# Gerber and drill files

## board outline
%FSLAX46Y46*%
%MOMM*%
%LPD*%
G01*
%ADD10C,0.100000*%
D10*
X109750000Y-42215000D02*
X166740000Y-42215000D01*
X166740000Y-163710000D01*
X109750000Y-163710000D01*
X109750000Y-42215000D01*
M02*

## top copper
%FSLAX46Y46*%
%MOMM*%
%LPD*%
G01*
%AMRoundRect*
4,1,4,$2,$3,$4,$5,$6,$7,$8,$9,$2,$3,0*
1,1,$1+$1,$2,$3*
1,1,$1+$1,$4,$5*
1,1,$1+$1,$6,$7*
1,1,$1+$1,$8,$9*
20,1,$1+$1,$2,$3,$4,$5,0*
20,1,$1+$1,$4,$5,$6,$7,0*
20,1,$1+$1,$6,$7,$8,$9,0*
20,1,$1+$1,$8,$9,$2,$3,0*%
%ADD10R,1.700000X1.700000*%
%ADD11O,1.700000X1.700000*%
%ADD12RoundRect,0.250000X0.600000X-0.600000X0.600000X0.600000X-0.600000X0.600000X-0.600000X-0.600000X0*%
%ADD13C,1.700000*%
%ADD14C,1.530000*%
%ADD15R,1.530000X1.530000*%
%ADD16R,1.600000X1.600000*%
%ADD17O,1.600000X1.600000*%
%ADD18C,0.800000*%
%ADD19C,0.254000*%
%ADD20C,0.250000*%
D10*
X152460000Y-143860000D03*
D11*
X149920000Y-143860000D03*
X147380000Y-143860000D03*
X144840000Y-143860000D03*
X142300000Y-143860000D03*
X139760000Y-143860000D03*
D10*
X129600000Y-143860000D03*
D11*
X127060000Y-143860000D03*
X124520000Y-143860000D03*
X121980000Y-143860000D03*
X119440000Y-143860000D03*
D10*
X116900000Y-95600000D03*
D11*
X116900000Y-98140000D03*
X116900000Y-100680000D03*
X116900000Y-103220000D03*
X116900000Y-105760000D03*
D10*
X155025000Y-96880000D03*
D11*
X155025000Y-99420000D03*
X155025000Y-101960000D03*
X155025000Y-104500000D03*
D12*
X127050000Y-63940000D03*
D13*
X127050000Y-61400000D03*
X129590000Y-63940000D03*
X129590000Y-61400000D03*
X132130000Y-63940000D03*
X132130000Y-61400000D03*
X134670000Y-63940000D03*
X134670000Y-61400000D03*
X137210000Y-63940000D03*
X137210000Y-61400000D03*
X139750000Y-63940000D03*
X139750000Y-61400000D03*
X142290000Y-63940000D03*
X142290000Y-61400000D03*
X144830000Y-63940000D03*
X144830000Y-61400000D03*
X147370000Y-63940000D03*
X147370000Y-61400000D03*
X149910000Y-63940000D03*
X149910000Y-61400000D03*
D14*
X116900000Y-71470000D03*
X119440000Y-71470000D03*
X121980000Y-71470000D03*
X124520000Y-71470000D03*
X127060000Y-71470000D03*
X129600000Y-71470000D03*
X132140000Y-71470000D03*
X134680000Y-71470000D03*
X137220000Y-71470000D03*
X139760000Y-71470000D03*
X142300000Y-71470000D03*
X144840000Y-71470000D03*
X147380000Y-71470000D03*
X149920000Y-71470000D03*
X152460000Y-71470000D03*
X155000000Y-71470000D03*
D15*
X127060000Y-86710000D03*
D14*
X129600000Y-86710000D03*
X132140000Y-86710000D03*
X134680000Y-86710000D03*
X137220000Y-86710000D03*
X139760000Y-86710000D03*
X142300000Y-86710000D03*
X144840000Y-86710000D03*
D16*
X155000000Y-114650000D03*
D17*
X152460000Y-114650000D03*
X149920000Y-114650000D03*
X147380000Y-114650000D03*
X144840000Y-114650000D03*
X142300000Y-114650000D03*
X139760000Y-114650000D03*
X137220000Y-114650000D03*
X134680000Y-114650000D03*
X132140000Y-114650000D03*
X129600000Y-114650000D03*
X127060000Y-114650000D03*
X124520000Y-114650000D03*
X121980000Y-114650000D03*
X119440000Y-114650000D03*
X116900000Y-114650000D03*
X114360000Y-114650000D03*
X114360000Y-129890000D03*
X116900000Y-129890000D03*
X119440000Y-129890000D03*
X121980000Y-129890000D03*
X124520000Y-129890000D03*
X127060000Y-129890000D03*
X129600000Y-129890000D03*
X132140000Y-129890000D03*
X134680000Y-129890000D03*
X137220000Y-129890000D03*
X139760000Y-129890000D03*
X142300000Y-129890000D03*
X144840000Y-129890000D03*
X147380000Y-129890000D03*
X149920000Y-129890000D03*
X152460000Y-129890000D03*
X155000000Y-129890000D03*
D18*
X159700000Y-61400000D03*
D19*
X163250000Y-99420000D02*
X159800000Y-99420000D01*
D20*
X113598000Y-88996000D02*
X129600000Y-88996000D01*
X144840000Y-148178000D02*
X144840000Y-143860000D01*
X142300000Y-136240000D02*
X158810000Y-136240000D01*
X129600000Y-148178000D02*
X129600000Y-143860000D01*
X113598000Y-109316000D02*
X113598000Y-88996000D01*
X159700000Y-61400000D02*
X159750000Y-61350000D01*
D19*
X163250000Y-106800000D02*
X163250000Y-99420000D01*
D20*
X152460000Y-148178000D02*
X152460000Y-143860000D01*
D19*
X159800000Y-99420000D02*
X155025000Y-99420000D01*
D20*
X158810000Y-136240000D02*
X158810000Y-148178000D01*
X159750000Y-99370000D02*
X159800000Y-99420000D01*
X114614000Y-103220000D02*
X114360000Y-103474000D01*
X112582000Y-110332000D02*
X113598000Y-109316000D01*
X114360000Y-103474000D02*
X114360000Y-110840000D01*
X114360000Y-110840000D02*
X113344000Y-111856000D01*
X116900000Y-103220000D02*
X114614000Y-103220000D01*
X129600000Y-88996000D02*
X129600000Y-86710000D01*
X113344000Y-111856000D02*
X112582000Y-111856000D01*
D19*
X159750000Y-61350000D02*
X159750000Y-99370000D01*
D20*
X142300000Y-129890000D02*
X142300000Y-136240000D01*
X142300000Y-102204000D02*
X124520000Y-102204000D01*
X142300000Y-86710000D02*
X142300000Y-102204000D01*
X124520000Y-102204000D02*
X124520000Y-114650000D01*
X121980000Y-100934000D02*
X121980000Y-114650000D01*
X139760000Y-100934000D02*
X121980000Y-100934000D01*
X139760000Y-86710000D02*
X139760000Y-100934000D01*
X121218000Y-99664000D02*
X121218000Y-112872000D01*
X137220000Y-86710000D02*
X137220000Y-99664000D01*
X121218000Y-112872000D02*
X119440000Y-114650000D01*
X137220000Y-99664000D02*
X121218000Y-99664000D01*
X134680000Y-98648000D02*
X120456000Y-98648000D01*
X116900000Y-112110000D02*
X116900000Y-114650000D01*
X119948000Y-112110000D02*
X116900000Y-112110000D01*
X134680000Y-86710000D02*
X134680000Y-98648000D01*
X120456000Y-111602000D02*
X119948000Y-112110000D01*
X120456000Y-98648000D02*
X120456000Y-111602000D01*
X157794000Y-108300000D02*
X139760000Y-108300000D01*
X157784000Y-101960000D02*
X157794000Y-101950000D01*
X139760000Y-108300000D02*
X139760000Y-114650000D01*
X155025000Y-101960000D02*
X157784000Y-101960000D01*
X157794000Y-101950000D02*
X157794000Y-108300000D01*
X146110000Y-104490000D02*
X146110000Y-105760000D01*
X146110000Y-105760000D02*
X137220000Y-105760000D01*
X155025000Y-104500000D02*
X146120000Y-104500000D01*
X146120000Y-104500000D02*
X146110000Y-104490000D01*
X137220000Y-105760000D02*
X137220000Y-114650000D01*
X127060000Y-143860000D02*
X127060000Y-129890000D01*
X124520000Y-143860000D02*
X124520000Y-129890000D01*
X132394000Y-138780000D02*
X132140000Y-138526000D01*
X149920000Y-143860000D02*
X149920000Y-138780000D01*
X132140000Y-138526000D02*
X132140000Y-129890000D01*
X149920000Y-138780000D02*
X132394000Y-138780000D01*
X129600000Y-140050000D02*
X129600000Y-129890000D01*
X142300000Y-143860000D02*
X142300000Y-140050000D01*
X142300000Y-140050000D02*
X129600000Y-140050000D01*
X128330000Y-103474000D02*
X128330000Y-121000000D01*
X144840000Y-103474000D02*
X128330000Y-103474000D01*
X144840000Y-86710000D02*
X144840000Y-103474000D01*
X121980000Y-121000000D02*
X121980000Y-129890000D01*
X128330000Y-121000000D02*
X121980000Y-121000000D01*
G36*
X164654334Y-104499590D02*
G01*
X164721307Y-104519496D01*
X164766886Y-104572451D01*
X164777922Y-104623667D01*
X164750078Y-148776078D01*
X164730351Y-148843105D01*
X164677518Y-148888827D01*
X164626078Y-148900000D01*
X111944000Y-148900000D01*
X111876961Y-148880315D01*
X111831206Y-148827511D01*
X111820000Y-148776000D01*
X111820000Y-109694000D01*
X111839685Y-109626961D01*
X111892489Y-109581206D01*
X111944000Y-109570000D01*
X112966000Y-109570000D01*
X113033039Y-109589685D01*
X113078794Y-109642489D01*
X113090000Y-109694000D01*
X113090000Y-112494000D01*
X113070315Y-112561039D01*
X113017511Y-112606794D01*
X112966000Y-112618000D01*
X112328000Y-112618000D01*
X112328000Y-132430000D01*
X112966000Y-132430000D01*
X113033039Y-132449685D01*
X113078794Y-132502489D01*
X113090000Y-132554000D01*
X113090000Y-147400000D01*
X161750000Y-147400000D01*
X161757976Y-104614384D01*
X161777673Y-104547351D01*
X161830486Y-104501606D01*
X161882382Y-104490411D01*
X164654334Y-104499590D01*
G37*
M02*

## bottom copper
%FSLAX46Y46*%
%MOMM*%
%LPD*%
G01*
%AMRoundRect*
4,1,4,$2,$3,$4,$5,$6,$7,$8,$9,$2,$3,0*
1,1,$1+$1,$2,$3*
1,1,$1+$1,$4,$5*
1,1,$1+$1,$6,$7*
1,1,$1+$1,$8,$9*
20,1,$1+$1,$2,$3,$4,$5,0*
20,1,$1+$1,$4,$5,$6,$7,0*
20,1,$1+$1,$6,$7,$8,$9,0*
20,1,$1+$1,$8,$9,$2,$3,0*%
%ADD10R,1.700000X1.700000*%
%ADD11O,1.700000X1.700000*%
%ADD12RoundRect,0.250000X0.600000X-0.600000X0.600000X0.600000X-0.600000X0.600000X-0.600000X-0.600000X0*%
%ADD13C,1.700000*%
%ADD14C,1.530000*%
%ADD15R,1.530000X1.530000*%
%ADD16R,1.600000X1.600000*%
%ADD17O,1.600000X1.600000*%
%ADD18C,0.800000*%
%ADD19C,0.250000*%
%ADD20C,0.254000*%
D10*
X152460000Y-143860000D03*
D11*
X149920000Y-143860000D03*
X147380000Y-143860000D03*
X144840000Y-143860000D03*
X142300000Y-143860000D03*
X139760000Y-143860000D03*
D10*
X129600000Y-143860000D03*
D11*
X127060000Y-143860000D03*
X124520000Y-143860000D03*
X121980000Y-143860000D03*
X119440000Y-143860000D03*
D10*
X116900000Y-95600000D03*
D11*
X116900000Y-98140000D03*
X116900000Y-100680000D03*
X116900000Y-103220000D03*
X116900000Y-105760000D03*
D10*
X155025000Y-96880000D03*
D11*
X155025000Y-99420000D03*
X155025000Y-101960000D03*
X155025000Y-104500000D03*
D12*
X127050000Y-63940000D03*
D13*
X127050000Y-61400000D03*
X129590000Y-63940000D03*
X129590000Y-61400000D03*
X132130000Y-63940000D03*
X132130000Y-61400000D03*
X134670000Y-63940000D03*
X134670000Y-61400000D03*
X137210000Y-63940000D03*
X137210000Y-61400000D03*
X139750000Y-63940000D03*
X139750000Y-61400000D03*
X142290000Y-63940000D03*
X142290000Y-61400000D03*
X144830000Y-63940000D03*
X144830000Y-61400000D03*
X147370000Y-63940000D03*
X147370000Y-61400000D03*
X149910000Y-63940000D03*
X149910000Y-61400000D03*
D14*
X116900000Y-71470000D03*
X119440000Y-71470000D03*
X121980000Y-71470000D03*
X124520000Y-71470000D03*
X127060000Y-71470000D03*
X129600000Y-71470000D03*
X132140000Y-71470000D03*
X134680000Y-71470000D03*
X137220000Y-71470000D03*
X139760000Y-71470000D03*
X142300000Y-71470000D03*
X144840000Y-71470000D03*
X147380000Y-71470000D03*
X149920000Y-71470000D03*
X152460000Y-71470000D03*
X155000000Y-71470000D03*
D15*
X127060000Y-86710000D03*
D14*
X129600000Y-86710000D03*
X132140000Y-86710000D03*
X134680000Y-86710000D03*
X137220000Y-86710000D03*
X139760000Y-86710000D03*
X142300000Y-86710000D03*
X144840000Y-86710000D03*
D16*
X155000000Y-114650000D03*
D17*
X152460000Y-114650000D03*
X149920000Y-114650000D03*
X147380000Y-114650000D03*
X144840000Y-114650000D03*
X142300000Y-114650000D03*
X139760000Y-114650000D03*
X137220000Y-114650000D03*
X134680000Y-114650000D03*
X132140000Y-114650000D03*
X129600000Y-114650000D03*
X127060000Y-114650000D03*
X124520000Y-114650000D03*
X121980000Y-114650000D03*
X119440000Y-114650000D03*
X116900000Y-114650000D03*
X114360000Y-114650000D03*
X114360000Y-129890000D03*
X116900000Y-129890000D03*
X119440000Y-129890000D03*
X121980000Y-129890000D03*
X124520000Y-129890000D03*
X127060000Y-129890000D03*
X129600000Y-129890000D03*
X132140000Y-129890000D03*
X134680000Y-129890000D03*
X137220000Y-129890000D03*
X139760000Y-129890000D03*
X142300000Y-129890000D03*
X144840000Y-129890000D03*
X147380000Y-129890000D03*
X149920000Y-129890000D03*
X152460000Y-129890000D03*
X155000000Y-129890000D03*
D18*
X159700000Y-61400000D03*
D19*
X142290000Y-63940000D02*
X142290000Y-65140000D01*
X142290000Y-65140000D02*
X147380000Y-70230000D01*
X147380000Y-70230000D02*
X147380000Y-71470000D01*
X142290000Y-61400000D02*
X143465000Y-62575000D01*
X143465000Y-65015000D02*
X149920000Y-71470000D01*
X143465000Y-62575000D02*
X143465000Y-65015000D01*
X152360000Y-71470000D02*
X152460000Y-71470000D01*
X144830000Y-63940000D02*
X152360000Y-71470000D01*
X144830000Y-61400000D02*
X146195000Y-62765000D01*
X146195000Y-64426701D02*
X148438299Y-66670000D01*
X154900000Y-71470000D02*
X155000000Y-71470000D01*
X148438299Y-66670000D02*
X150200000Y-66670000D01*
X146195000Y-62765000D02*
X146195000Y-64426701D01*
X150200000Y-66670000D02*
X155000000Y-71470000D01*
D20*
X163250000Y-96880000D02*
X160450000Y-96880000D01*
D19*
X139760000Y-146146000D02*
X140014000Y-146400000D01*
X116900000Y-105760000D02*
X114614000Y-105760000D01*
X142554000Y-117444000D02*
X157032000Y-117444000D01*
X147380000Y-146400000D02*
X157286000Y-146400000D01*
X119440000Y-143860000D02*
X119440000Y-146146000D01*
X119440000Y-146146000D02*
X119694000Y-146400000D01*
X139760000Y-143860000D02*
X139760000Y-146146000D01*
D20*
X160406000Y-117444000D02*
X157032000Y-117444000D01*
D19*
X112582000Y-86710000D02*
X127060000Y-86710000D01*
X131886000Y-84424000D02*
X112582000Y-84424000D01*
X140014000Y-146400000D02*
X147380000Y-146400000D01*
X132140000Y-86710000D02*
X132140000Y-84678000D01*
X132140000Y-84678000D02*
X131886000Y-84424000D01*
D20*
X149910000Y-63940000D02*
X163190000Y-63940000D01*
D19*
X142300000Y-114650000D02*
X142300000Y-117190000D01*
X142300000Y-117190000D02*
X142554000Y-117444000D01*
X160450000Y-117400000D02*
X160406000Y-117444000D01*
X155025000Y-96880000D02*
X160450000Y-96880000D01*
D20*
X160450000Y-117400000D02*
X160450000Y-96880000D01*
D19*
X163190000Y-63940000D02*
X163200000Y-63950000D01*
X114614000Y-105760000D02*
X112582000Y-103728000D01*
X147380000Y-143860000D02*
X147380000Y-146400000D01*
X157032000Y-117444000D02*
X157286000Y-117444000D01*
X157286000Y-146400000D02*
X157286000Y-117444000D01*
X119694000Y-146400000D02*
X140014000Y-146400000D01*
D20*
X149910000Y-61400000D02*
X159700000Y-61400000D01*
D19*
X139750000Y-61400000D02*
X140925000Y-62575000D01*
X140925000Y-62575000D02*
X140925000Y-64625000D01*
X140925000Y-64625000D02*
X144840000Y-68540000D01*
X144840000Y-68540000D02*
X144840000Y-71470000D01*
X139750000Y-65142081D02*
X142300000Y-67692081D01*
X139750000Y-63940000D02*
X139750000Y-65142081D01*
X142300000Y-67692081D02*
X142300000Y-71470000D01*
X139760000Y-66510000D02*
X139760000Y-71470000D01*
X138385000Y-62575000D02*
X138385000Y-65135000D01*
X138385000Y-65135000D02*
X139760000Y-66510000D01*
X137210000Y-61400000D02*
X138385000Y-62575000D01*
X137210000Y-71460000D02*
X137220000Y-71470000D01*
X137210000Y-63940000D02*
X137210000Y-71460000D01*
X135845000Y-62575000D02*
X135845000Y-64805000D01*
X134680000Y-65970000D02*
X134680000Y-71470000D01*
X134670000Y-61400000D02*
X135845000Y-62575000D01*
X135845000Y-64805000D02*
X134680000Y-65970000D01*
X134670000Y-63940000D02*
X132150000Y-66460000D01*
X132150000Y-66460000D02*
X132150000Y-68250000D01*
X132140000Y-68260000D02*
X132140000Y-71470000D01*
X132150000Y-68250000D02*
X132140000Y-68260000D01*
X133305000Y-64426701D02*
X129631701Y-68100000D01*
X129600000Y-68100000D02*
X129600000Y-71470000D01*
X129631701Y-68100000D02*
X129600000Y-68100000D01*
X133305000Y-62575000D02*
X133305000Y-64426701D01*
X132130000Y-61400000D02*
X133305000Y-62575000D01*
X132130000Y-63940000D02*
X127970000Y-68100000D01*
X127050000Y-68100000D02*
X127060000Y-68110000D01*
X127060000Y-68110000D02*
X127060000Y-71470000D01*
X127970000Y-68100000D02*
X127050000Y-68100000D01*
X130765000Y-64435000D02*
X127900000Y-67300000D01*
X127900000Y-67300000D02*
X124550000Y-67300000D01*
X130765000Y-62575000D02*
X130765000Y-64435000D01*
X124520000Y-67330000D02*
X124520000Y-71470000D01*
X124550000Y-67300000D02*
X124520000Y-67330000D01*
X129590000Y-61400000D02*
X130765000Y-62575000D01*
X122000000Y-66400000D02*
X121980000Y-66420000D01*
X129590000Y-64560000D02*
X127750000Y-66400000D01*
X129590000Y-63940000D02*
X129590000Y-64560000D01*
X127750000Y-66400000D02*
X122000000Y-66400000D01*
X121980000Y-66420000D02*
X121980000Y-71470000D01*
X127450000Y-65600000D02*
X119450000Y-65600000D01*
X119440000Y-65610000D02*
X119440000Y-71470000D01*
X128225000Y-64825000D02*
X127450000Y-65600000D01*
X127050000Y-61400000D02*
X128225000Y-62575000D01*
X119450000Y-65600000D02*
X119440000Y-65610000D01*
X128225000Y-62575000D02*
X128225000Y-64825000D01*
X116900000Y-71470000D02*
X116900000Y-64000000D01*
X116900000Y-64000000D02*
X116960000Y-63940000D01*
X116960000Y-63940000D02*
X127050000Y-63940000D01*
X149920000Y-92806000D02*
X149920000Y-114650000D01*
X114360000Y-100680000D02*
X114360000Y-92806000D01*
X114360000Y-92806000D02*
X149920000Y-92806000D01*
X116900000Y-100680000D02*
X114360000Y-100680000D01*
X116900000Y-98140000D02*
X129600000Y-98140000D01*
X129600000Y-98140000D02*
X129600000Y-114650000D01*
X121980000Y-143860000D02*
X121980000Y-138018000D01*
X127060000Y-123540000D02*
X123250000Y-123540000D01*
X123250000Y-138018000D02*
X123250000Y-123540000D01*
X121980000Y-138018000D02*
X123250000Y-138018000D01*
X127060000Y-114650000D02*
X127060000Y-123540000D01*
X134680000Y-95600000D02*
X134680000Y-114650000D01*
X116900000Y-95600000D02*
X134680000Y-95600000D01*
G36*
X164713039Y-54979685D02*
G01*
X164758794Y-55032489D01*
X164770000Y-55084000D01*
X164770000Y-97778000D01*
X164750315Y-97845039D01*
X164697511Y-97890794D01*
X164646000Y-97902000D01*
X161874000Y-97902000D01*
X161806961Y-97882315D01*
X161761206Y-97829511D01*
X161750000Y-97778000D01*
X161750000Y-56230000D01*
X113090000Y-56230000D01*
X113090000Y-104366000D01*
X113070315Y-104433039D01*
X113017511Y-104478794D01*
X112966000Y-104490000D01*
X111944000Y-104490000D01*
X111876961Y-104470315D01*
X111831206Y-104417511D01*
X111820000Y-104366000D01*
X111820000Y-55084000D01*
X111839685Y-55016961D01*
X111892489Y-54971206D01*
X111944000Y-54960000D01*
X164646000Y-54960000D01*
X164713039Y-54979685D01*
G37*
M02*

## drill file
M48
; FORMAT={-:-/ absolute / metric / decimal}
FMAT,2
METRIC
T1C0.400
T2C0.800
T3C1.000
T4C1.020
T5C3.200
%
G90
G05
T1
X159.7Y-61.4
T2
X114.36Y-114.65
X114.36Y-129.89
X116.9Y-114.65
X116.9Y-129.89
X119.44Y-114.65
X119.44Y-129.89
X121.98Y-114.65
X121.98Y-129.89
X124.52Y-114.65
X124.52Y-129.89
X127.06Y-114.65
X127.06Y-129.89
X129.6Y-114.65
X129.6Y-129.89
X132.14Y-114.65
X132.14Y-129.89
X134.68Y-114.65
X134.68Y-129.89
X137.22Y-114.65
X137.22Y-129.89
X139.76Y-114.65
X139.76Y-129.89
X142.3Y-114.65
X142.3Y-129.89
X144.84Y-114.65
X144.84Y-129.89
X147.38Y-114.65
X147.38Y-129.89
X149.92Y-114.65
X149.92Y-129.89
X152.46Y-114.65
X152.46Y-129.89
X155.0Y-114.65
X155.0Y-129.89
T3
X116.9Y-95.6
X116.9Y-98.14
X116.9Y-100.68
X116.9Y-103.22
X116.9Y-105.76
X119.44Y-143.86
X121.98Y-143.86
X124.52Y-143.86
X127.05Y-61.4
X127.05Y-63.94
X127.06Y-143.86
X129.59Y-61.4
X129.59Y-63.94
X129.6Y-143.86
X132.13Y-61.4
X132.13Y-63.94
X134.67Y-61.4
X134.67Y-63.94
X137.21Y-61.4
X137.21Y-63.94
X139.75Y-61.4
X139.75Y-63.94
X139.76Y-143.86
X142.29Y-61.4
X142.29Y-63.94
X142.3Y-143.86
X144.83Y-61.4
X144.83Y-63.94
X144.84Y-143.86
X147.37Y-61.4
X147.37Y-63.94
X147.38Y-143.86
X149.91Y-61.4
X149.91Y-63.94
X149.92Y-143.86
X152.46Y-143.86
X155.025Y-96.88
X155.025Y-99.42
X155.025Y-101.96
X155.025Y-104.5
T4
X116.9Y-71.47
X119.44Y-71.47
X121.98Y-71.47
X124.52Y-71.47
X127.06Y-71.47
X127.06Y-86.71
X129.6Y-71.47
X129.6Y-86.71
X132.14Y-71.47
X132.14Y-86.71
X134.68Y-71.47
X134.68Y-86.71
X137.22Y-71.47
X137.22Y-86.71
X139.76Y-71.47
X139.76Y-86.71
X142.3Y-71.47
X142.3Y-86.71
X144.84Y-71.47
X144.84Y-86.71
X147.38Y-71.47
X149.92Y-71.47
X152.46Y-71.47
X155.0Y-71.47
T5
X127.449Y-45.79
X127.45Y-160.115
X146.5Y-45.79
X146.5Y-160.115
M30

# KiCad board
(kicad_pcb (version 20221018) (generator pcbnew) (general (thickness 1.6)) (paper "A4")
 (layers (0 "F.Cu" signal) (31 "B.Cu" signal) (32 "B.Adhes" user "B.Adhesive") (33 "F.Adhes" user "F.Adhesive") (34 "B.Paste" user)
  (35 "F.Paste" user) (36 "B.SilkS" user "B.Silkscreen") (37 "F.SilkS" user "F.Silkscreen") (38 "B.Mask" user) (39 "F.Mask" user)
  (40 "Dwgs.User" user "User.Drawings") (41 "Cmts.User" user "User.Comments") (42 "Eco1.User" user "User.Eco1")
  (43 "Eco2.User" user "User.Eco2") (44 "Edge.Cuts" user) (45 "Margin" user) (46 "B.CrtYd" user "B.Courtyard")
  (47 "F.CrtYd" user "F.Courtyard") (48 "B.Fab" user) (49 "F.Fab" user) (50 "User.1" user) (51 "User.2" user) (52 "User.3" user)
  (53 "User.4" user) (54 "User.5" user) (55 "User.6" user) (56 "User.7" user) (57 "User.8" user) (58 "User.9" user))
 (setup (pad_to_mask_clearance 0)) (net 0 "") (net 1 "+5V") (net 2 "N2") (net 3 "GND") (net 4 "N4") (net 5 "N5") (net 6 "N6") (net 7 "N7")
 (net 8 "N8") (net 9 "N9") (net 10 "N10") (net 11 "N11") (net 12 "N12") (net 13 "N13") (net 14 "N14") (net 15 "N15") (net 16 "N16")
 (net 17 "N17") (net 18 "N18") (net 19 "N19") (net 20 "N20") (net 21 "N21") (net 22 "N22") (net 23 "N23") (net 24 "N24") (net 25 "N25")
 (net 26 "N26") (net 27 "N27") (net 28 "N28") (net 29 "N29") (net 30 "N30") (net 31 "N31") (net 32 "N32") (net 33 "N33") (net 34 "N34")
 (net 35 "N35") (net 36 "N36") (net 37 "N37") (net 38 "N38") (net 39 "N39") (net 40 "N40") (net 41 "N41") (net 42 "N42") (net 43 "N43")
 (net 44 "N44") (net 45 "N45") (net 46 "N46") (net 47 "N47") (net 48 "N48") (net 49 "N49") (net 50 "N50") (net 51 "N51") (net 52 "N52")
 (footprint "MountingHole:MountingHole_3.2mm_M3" (layer "F.Cu") (at 127.448582 45.79)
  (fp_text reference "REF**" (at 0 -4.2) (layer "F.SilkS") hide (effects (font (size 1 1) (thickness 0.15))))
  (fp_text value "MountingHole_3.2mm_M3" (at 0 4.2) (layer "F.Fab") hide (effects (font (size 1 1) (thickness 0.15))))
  (pad "" np_thru_hole circle (at 0 0) (size 3.2 3.2) (drill 3.2) (layers "*.Cu" "*.Mask")))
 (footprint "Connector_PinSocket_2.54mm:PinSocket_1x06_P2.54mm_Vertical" (layer "F.Cu") (at 152.46 143.86 -90)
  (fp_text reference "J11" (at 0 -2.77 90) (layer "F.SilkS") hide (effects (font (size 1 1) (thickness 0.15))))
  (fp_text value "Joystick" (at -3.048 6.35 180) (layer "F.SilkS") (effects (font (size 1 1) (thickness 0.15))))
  (pad "1" thru_hole rect (at 0 0 270) (size 1.7 1.7) (drill 1) (layers "*.Cu" "*.Mask") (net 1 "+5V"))
  (pad "2" thru_hole oval (at 0 2.54 270) (size 1.7 1.7) (drill 1) (layers "*.Cu" "*.Mask") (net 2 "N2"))
  (pad "3" thru_hole oval (at 0 5.08 270) (size 1.7 1.7) (drill 1) (layers "*.Cu" "*.Mask") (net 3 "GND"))
  (pad "4" thru_hole oval (at 0 7.62 270) (size 1.7 1.7) (drill 1) (layers "*.Cu" "*.Mask") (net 1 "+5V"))
  (pad "5" thru_hole oval (at 0 10.16 270) (size 1.7 1.7) (drill 1) (layers "*.Cu" "*.Mask") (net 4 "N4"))
  (pad "6" thru_hole oval (at 0 12.7 270) (size 1.7 1.7) (drill 1) (layers "*.Cu" "*.Mask") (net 3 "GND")))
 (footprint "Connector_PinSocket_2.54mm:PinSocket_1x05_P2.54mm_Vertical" (layer "F.Cu") (at 129.6 143.86 -90)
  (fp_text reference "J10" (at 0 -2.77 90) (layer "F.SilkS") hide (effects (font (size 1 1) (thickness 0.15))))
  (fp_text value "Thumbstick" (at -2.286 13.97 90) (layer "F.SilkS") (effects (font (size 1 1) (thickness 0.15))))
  (pad "1" thru_hole rect (at 0 0 270) (size 1.7 1.7) (drill 1) (layers "*.Cu" "*.Mask") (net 1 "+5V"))
  (pad "2" thru_hole oval (at 0 2.54 270) (size 1.7 1.7) (drill 1) (layers "*.Cu" "*.Mask") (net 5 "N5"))
  (pad "3" thru_hole oval (at 0 5.08 270) (size 1.7 1.7) (drill 1) (layers "*.Cu" "*.Mask") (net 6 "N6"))
  (pad "4" thru_hole oval (at 0 7.62 270) (size 1.7 1.7) (drill 1) (layers "*.Cu" "*.Mask") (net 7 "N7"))
  (pad "5" thru_hole oval (at 0 10.16 270) (size 1.7 1.7) (drill 1) (layers "*.Cu" "*.Mask") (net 3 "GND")))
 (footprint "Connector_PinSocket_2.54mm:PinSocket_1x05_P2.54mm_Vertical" (layer "F.Cu") (at 116.9 95.6)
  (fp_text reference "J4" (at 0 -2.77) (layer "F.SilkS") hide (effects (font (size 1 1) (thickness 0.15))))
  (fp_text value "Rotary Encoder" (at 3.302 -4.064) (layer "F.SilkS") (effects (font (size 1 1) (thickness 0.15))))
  (pad "1" thru_hole rect (at 0 0) (size 1.7 1.7) (drill 1) (layers "*.Cu" "*.Mask") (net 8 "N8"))
  (pad "2" thru_hole oval (at 0 2.54) (size 1.7 1.7) (drill 1) (layers "*.Cu" "*.Mask") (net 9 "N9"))
  (pad "3" thru_hole oval (at 0 5.08) (size 1.7 1.7) (drill 1) (layers "*.Cu" "*.Mask") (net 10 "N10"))
  (pad "4" thru_hole oval (at 0 7.62) (size 1.7 1.7) (drill 1) (layers "*.Cu" "*.Mask") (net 1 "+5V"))
  (pad "5" thru_hole oval (at 0 10.16) (size 1.7 1.7) (drill 1) (layers "*.Cu" "*.Mask") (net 3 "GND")))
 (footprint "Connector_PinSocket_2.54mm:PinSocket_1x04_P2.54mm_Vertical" (layer "F.Cu") (at 155.025 96.88)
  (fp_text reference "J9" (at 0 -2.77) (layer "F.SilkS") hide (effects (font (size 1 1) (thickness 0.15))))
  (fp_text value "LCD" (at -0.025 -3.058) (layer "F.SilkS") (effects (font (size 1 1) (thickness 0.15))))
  (pad "1" thru_hole rect (at 0 0) (size 1.7 1.7) (drill 1) (layers "*.Cu" "*.Mask") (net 3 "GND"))
  (pad "2" thru_hole oval (at 0 2.54) (size 1.7 1.7) (drill 1) (layers "*.Cu" "*.Mask") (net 1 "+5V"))
  (pad "3" thru_hole oval (at 0 5.08) (size 1.7 1.7) (drill 1) (layers "*.Cu" "*.Mask") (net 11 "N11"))
  (pad "4" thru_hole oval (at 0 7.62) (size 1.7 1.7) (drill 1) (layers "*.Cu" "*.Mask") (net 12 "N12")))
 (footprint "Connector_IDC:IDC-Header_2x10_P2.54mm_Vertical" (layer "F.Cu") (at 127.05 63.94 90)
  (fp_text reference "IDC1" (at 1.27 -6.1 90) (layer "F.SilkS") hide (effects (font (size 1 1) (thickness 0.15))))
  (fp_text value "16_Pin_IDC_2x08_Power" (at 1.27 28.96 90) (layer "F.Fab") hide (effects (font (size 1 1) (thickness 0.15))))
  (pad "1" thru_hole roundrect (at 0 0 90) (size 1.7 1.7) (drill 1) (layers "*.Cu" "*.Mask") (roundrect_rratio 0.1470588235) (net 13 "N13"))
  (pad "2" thru_hole circle (at 2.54 0 90) (size 1.7 1.7) (drill 1) (layers "*.Cu" "*.Mask") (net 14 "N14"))
  (pad "3" thru_hole circle (at 0 2.54 90) (size 1.7 1.7) (drill 1) (layers "*.Cu" "*.Mask") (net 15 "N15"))
  (pad "4" thru_hole circle (at 2.54 2.54 90) (size 1.7 1.7) (drill 1) (layers "*.Cu" "*.Mask") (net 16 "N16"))
  (pad "5" thru_hole circle (at 0 5.08 90) (size 1.7 1.7) (drill 1) (layers "*.Cu" "*.Mask") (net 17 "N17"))
  (pad "6" thru_hole circle (at 2.54 5.08 90) (size 1.7 1.7) (drill 1) (layers "*.Cu" "*.Mask") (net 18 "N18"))
  (pad "7" thru_hole circle (at 0 7.62 90) (size 1.7 1.7) (drill 1) (layers "*.Cu" "*.Mask") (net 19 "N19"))
  (pad "8" thru_hole circle (at 2.54 7.62 90) (size 1.7 1.7) (drill 1) (layers "*.Cu" "*.Mask") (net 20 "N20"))
  (pad "9" thru_hole circle (at 0 10.16 90) (size 1.7 1.7) (drill 1) (layers "*.Cu" "*.Mask") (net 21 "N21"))
  (pad "10" thru_hole circle (at 2.54 10.16 90) (size 1.7 1.7) (drill 1) (layers "*.Cu" "*.Mask") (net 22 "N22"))
  (pad "11" thru_hole circle (at 0 12.7 90) (size 1.7 1.7) (drill 1) (layers "*.Cu" "*.Mask") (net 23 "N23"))
  (pad "12" thru_hole circle (at 2.54 12.7 90) (size 1.7 1.7) (drill 1) (layers "*.Cu" "*.Mask") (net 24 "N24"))
  (pad "13" thru_hole circle (at 0 15.24 90) (size 1.7 1.7) (drill 1) (layers "*.Cu" "*.Mask") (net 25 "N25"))
  (pad "14" thru_hole circle (at 2.54 15.24 90) (size 1.7 1.7) (drill 1) (layers "*.Cu" "*.Mask") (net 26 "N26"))
  (pad "15" thru_hole circle (at 0 17.78 90) (size 1.7 1.7) (drill 1) (layers "*.Cu" "*.Mask") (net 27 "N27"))
  (pad "16" thru_hole circle (at 2.54 17.78 90) (size 1.7 1.7) (drill 1) (layers "*.Cu" "*.Mask") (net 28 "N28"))
  (pad "17" thru_hole circle (at 0 20.32 90) (size 1.7 1.7) (drill 1) (layers "*.Cu" "*.Mask") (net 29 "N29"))
  (pad "18" thru_hole circle (at 2.54 20.32 90) (size 1.7 1.7) (drill 1) (layers "*.Cu" "*.Mask") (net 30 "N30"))
  (pad "19" thru_hole circle (at 0 22.86 90) (size 1.7 1.7) (drill 1) (layers "*.Cu" "*.Mask") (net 3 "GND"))
  (pad "20" thru_hole circle (at 2.54 22.86 90) (size 1.7 1.7) (drill 1) (layers "*.Cu" "*.Mask") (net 1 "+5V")))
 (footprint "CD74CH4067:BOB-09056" (layer "F.Cu") (at 135.95 79.09 -90)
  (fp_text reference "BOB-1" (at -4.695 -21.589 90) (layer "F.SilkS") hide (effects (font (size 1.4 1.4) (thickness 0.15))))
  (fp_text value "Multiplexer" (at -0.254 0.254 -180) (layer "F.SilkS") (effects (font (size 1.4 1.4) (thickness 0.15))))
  (pad "JP1-1" thru_hole circle (at -7.62 19.05 270) (size 1.53 1.53) (drill 1.02) (layers "*.Cu" "*.Mask") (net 13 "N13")
   (solder_mask_margin 0.102))
  (pad "JP1-2" thru_hole circle (at -7.62 16.51 270) (size 1.53 1.53) (drill 1.02) (layers "*.Cu" "*.Mask") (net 14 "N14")
   (solder_mask_margin 0.102))
  (pad "JP1-3" thru_hole circle (at -7.62 13.97 270) (size 1.53 1.53) (drill 1.02) (layers "*.Cu" "*.Mask") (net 15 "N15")
   (solder_mask_margin 0.102))
  (pad "JP1-4" thru_hole circle (at -7.62 11.43 270) (size 1.53 1.53) (drill 1.02) (layers "*.Cu" "*.Mask") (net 16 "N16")
   (solder_mask_margin 0.102))
  (pad "JP1-5" thru_hole circle (at -7.62 8.89 270) (size 1.53 1.53) (drill 1.02) (layers "*.Cu" "*.Mask") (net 17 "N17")
   (solder_mask_margin 0.102))
  (pad "JP1-6" thru_hole circle (at -7.62 6.35 270) (size 1.53 1.53) (drill 1.02) (layers "*.Cu" "*.Mask") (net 18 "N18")
   (solder_mask_margin 0.102))
  (pad "JP1-7" thru_hole circle (at -7.62 3.81 270) (size 1.53 1.53) (drill 1.02) (layers "*.Cu" "*.Mask") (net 19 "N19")
   (solder_mask_margin 0.102))
  (pad "JP1-8" thru_hole circle (at -7.62 1.27 270) (size 1.53 1.53) (drill 1.02) (layers "*.Cu" "*.Mask") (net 20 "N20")
   (solder_mask_margin 0.102))
  (pad "JP1-9" thru_hole circle (at -7.62 -1.27 270) (size 1.53 1.53) (drill 1.02) (layers "*.Cu" "*.Mask") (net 21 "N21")
   (solder_mask_margin 0.102))
  (pad "JP1-10" thru_hole circle (at -7.62 -3.81 270) (size 1.53 1.53) (drill 1.02) (layers "*.Cu" "*.Mask") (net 22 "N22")
   (solder_mask_margin 0.102))
  (pad "JP1-11" thru_hole circle (at -7.62 -6.35 270) (size 1.53 1.53) (drill 1.02) (layers "*.Cu" "*.Mask") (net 23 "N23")
   (solder_mask_margin 0.102))
  (pad "JP1-12" thru_hole circle (at -7.62 -8.89 270) (size 1.53 1.53) (drill 1.02) (layers "*.Cu" "*.Mask") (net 24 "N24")
   (solder_mask_margin 0.102))
  (pad "JP1-13" thru_hole circle (at -7.62 -11.43 270) (size 1.53 1.53) (drill 1.02) (layers "*.Cu" "*.Mask") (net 25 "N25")
   (solder_mask_margin 0.102))
  (pad "JP1-14" thru_hole circle (at -7.62 -13.97 270) (size 1.53 1.53) (drill 1.02) (layers "*.Cu" "*.Mask") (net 26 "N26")
   (solder_mask_margin 0.102))
  (pad "JP1-15" thru_hole circle (at -7.62 -16.51 270) (size 1.53 1.53) (drill 1.02) (layers "*.Cu" "*.Mask") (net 27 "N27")
   (solder_mask_margin 0.102))
  (pad "JP1-16" thru_hole circle (at -7.62 -19.05 270) (size 1.53 1.53) (drill 1.02) (layers "*.Cu" "*.Mask") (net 28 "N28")
   (solder_mask_margin 0.102))
  (pad "JP3-1" thru_hole rect (at 7.62 8.89 270) (size 1.53 1.53) (drill 1.02) (layers "*.Cu" "*.Mask") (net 3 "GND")
   (solder_mask_margin 0.102))
  (pad "JP3-2" thru_hole circle (at 7.62 6.35 270) (size 1.53 1.53) (drill 1.02) (layers "*.Cu" "*.Mask") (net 1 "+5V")
   (solder_mask_margin 0.102))
  (pad "JP3-3" thru_hole circle (at 7.62 3.81 270) (size 1.53 1.53) (drill 1.02) (layers "*.Cu" "*.Mask") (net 3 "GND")
   (solder_mask_margin 0.102))
  (pad "JP3-4" thru_hole circle (at 7.62 1.27 270) (size 1.53 1.53) (drill 1.02) (layers "*.Cu" "*.Mask") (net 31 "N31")
   (solder_mask_margin 0.102))
  (pad "JP3-5" thru_hole circle (at 7.62 -1.27 270) (size 1.53 1.53) (drill 1.02) (layers "*.Cu" "*.Mask") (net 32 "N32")
   (solder_mask_margin 0.102))
  (pad "JP3-6" thru_hole circle (at 7.62 -3.81 270) (size 1.53 1.53) (drill 1.02) (layers "*.Cu" "*.Mask") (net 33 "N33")
   (solder_mask_margin 0.102))
  (pad "JP3-7" thru_hole circle (at 7.62 -6.35 270) (size 1.53 1.53) (drill 1.02) (layers "*.Cu" "*.Mask") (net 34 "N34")
   (solder_mask_margin 0.102))
  (pad "JP3-8" thru_hole circle (at 7.62 -8.89 270) (size 1.53 1.53) (drill 1.02) (layers "*.Cu" "*.Mask") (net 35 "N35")
   (solder_mask_margin 0.102)))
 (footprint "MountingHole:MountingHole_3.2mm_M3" (layer "F.Cu") (at 146.5 160.115)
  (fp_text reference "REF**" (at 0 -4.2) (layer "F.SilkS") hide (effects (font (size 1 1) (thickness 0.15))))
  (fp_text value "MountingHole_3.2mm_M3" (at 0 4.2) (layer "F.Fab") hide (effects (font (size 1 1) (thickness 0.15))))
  (pad "" np_thru_hole circle (at 0 0) (size 3.2 3.2) (drill 3.2) (layers "*.Cu" "*.Mask")))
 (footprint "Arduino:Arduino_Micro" (layer "F.Cu") (at 155 114.65 -90)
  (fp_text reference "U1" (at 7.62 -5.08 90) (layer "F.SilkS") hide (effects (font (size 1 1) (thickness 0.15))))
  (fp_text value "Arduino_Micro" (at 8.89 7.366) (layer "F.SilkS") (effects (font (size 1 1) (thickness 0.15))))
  (pad "1" thru_hole rect (at 0 0 270) (size 1.6 1.6) (drill 0.8) (layers "*.Cu" "*.Mask") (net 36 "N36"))
  (pad "2" thru_hole oval (at 0 2.54 270) (size 1.6 1.6) (drill 0.8) (layers "*.Cu" "*.Mask") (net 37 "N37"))
  (pad "3" thru_hole oval (at 0 5.08 270) (size 1.6 1.6) (drill 0.8) (layers "*.Cu" "*.Mask") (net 10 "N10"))
  (pad "4" thru_hole oval (at 0 7.62 270) (size 1.6 1.6) (drill 0.8) (layers "*.Cu" "*.Mask") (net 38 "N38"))
  (pad "5" thru_hole oval (at 0 10.16 270) (size 1.6 1.6) (drill 0.8) (layers "*.Cu" "*.Mask") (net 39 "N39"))
  (pad "6" thru_hole oval (at 0 12.7 270) (size 1.6 1.6) (drill 0.8) (layers "*.Cu" "*.Mask") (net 3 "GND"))
  (pad "7" thru_hole oval (at 0 15.24 270) (size 1.6 1.6) (drill 0.8) (layers "*.Cu" "*.Mask") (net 11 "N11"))
  (pad "8" thru_hole oval (at 0 17.78 270) (size 1.6 1.6) (drill 0.8) (layers "*.Cu" "*.Mask") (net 12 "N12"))
  (pad "9" thru_hole oval (at 0 20.32 270) (size 1.6 1.6) (drill 0.8) (layers "*.Cu" "*.Mask") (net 8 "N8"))
  (pad "10" thru_hole oval (at 0 22.86 270) (size 1.6 1.6) (drill 0.8) (layers "*.Cu" "*.Mask") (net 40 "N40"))
  (pad "11" thru_hole oval (at 0 25.4 270) (size 1.6 1.6) (drill 0.8) (layers "*.Cu" "*.Mask") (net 9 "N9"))
  (pad "12" thru_hole oval (at 0 27.94 270) (size 1.6 1.6) (drill 0.8) (layers "*.Cu" "*.Mask") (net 7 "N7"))
  (pad "13" thru_hole oval (at 0 30.48 270) (size 1.6 1.6) (drill 0.8) (layers "*.Cu" "*.Mask") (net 34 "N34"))
  (pad "14" thru_hole oval (at 0 33.02 270) (size 1.6 1.6) (drill 0.8) (layers "*.Cu" "*.Mask") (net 33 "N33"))
  (pad "15" thru_hole oval (at 0 35.56 270) (size 1.6 1.6) (drill 0.8) (layers "*.Cu" "*.Mask") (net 32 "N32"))
  (pad "16" thru_hole oval (at 0 38.1 270) (size 1.6 1.6) (drill 0.8) (layers "*.Cu" "*.Mask") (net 31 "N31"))
  (pad "17" thru_hole oval (at 0 40.64 270) (size 1.6 1.6) (drill 0.8) (layers "*.Cu" "*.Mask") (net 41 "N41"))
  (pad "18" thru_hole oval (at 15.24 40.64 270) (size 1.6 1.6) (drill 0.8) (layers "*.Cu" "*.Mask") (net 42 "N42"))
  (pad "19" thru_hole oval (at 15.24 38.1 270) (size 1.6 1.6) (drill 0.8) (layers "*.Cu" "*.Mask") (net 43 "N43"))
  (pad "20" thru_hole oval (at 15.24 35.56 270) (size 1.6 1.6) (drill 0.8) (layers "*.Cu" "*.Mask") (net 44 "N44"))
  (pad "21" thru_hole oval (at 15.24 33.02 270) (size 1.6 1.6) (drill 0.8) (layers "*.Cu" "*.Mask") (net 35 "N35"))
  (pad "22" thru_hole oval (at 15.24 30.48 270) (size 1.6 1.6) (drill 0.8) (layers "*.Cu" "*.Mask") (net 6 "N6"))
  (pad "23" thru_hole oval (at 15.24 27.94 270) (size 1.6 1.6) (drill 0.8) (layers "*.Cu" "*.Mask") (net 5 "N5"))
  (pad "24" thru_hole oval (at 15.24 25.4 270) (size 1.6 1.6) (drill 0.8) (layers "*.Cu" "*.Mask") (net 4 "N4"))
  (pad "25" thru_hole oval (at 15.24 22.86 270) (size 1.6 1.6) (drill 0.8) (layers "*.Cu" "*.Mask") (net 2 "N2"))
  (pad "26" thru_hole oval (at 15.24 20.32 270) (size 1.6 1.6) (drill 0.8) (layers "*.Cu" "*.Mask") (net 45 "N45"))
  (pad "27" thru_hole oval (at 15.24 17.78 270) (size 1.6 1.6) (drill 0.8) (layers "*.Cu" "*.Mask") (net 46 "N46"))
  (pad "28" thru_hole oval (at 15.24 15.24 270) (size 1.6 1.6) (drill 0.8) (layers "*.Cu" "*.Mask") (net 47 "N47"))
  (pad "29" thru_hole oval (at 15.24 12.7 270) (size 1.6 1.6) (drill 0.8) (layers "*.Cu" "*.Mask") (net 1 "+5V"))
  (pad "30" thru_hole oval (at 15.24 10.16 270) (size 1.6 1.6) (drill 0.8) (layers "*.Cu" "*.Mask") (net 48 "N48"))
  (pad "31" thru_hole oval (at 15.24 7.62 270) (size 1.6 1.6) (drill 0.8) (layers "*.Cu" "*.Mask") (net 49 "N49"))
  (pad "32" thru_hole oval (at 15.24 5.08 270) (size 1.6 1.6) (drill 0.8) (layers "*.Cu" "*.Mask") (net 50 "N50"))
  (pad "33" thru_hole oval (at 15.24 2.54 270) (size 1.6 1.6) (drill 0.8) (layers "*.Cu" "*.Mask") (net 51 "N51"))
  (pad "34" thru_hole oval (at 15.24 0 270) (size 1.6 1.6) (drill 0.8) (layers "*.Cu" "*.Mask") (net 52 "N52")))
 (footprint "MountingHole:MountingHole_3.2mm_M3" (layer "F.Cu") (at 127.45 160.115)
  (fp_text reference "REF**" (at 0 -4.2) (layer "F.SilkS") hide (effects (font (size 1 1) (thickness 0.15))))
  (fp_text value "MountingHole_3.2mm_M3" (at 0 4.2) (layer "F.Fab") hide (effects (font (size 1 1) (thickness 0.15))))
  (pad "" np_thru_hole circle (at 0 0) (size 3.2 3.2) (drill 3.2) (layers "*.Cu" "*.Mask")))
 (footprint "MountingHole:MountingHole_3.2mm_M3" (layer "F.Cu") (at 146.5 45.79)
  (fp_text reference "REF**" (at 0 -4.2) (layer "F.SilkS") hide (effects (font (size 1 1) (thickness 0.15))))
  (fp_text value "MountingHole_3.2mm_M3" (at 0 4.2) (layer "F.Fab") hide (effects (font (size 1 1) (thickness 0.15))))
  (pad "" np_thru_hole circle (at 0 0) (size 3.2 3.2) (drill 3.2) (layers "*.Cu" "*.Mask")))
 (gr_rect (start 109.75 42.215) (end 166.74 163.71) (stroke (width 0.1) (type default)) (fill none) (layer "Edge.Cuts"))
 (segment (start 142.29 63.94) (end 142.29 65.14) (width 0.25) (layer "B.Cu") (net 25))
 (segment (start 142.29 65.14) (end 147.38 70.23) (width 0.25) (layer "B.Cu") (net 25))
 (segment (start 147.38 70.23) (end 147.38 71.47) (width 0.25) (layer "B.Cu") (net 25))
 (segment (start 142.29 61.4) (end 143.465 62.575) (width 0.25) (layer "B.Cu") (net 26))
 (segment (start 143.465 65.015) (end 149.92 71.47) (width 0.25) (layer "B.Cu") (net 26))
 (segment (start 143.465 62.575) (end 143.465 65.015) (width 0.25) (layer "B.Cu") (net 26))
 (segment (start 152.36 71.47) (end 152.46 71.47) (width 0.25) (layer "B.Cu") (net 27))
 (segment (start 144.83 63.94) (end 152.36 71.47) (width 0.25) (layer "B.Cu") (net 27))
 (segment (start 144.83 61.4) (end 146.195 62.765) (width 0.25) (layer "B.Cu") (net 28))
 (segment (start 146.195 64.426701) (end 148.438299 66.67) (width 0.25) (layer "B.Cu") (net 28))
 (segment (start 154.9 71.47) (end 155 71.47) (width 0.25) (layer "B.Cu") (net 28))
 (segment (start 148.438299 66.67) (end 150.2 66.67) (width 0.25) (layer "B.Cu") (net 28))
 (segment (start 146.195 62.765) (end 146.195 64.426701) (width 0.25) (layer "B.Cu") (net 28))
 (segment (start 150.2 66.67) (end 155 71.47) (width 0.25) (layer "B.Cu") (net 28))
 (segment (start 163.25 96.88) (end 160.45 96.88) (width 0.254) (layer "B.Cu") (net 3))
 (segment (start 139.76 146.146) (end 140.014 146.4) (width 0.25) (layer "B.Cu") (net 3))
 (segment (start 116.9 105.76) (end 114.614 105.76) (width 0.25) (layer "B.Cu") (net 3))
 (segment (start 142.554 117.444) (end 157.032 117.444) (width 0.25) (layer "B.Cu") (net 3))
 (segment (start 147.38 146.4) (end 157.286 146.4) (width 0.25) (layer "B.Cu") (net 3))
 (segment (start 119.44 143.86) (end 119.44 146.146) (width 0.25) (layer "B.Cu") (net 3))
 (segment (start 119.44 146.146) (end 119.694 146.4) (width 0.25) (layer "B.Cu") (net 3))
 (segment (start 139.76 143.86) (end 139.76 146.146) (width 0.25) (layer "B.Cu") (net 3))
 (segment (start 160.406 117.444) (end 157.032 117.444) (width 0.254) (layer "B.Cu") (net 3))
 (segment (start 112.582 86.71) (end 127.06 86.71) (width 0.25) (layer "B.Cu") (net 3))
 (segment (start 131.886 84.424) (end 112.582 84.424) (width 0.25) (layer "B.Cu") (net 3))
 (segment (start 140.014 146.4) (end 147.38 146.4) (width 0.25) (layer "B.Cu") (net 3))
 (segment (start 132.14 86.71) (end 132.14 84.678) (width 0.25) (layer "B.Cu") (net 3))
 (segment (start 132.14 84.678) (end 131.886 84.424) (width 0.25) (layer "B.Cu") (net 3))
 (segment (start 149.91 63.94) (end 163.19 63.94) (width 0.254) (layer "B.Cu") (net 3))
 (segment (start 142.3 114.65) (end 142.3 117.19) (width 0.25) (layer "B.Cu") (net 3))
 (segment (start 142.3 117.19) (end 142.554 117.444) (width 0.25) (layer "B.Cu") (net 3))
 (segment (start 160.45 117.4) (end 160.406 117.444) (width 0.25) (layer "B.Cu") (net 3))
 (segment (start 155.025 96.88) (end 160.45 96.88) (width 0.25) (layer "B.Cu") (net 3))
 (segment (start 160.45 117.4) (end 160.45 96.88) (width 0.254) (layer "B.Cu") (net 3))
 (segment (start 163.19 63.94) (end 163.2 63.95) (width 0.25) (layer "B.Cu") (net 3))
 (segment (start 114.614 105.76) (end 112.582 103.728) (width 0.25) (layer "B.Cu") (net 3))
 (segment (start 147.38 143.86) (end 147.38 146.4) (width 0.25) (layer "B.Cu") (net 3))
 (segment (start 157.032 117.444) (end 157.286 117.444) (width 0.25) (layer "B.Cu") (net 3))
 (segment (start 157.286 146.4) (end 157.286 117.444) (width 0.25) (layer "B.Cu") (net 3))
 (segment (start 119.694 146.4) (end 140.014 146.4) (width 0.25) (layer "B.Cu") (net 3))
 (segment (start 163.25 99.42) (end 159.8 99.42) (width 0.254) (layer "F.Cu") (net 1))
 (segment (start 113.598 88.996) (end 129.6 88.996) (width 0.25) (layer "F.Cu") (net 1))
 (segment (start 144.84 148.178) (end 144.84 143.86) (width 0.25) (layer "F.Cu") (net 1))
 (segment (start 142.3 136.24) (end 158.81 136.24) (width 0.25) (layer "F.Cu") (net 1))
 (segment (start 129.6 148.178) (end 129.6 143.86) (width 0.25) (layer "F.Cu") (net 1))
 (segment (start 113.598 109.316) (end 113.598 88.996) (width 0.25) (layer "F.Cu") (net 1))
 (segment (start 159.7 61.4) (end 159.75 61.35) (width 0.25) (layer "F.Cu") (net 1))
 (segment (start 163.25 106.8) (end 163.25 99.42) (width 0.254) (layer "F.Cu") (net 1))
 (segment (start 152.46 148.178) (end 152.46 143.86) (width 0.25) (layer "F.Cu") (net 1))
 (segment (start 159.8 99.42) (end 155.025 99.42) (width 0.254) (layer "F.Cu") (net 1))
 (segment (start 158.81 136.24) (end 158.81 148.178) (width 0.25) (layer "F.Cu") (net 1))
 (segment (start 159.75 99.37) (end 159.8 99.42) (width 0.25) (layer "F.Cu") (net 1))
 (segment (start 114.614 103.22) (end 114.36 103.474) (width 0.25) (layer "F.Cu") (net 1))
 (segment (start 112.582 110.332) (end 113.598 109.316) (width 0.25) (layer "F.Cu") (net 1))
 (segment (start 114.36 103.474) (end 114.36 110.84) (width 0.25) (layer "F.Cu") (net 1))
 (segment (start 114.36 110.84) (end 113.344 111.856) (width 0.25) (layer "F.Cu") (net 1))
 (segment (start 116.9 103.22) (end 114.614 103.22) (width 0.25) (layer "F.Cu") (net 1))
 (segment (start 129.6 88.996) (end 129.6 86.71) (width 0.25) (layer "F.Cu") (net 1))
 (segment (start 113.344 111.856) (end 112.582 111.856) (width 0.25) (layer "F.Cu") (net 1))
 (segment (start 159.75 61.35) (end 159.75 99.37) (width 0.254) (layer "F.Cu") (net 1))
 (segment (start 142.3 129.89) (end 142.3 136.24) (width 0.25) (layer "F.Cu") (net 1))
 (via (at 159.7 61.4) (size 0.8) (drill 0.4) (layers "F.Cu" "B.Cu") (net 1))
 (segment (start 149.91 61.4) (end 159.7 61.4) (width 0.254) (layer "B.Cu") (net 1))
 (segment (start 139.75 61.4) (end 140.925 62.575) (width 0.25) (layer "B.Cu") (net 24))
 (segment (start 140.925 62.575) (end 140.925 64.625) (width 0.25) (layer "B.Cu") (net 24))
 (segment (start 140.925 64.625) (end 144.84 68.54) (width 0.25) (layer "B.Cu") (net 24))
 (segment (start 144.84 68.54) (end 144.84 71.47) (width 0.25) (layer "B.Cu") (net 24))
 (segment (start 139.75 65.142081) (end 142.3 67.692081) (width 0.25) (layer "B.Cu") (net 23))
 (segment (start 139.75 63.94) (end 139.75 65.142081) (width 0.25) (layer "B.Cu") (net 23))
 (segment (start 142.3 67.692081) (end 142.3 71.47) (width 0.25) (layer "B.Cu") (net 23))
 (segment (start 139.76 66.51) (end 139.76 71.47) (width 0.25) (layer "B.Cu") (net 22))
 (segment (start 138.385 62.575) (end 138.385 65.135) (width 0.25) (layer "B.Cu") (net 22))
 (segment (start 138.385 65.135) (end 139.76 66.51) (width 0.25) (layer "B.Cu") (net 22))
 (segment (start 137.21 61.4) (end 138.385 62.575) (width 0.25) (layer "B.Cu") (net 22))
 (segment (start 137.21 71.46) (end 137.22 71.47) (width 0.25) (layer "B.Cu") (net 21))
 (segment (start 137.21 63.94) (end 137.21 71.46) (width 0.25) (layer "B.Cu") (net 21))
 (segment (start 135.845 62.575) (end 135.845 64.805) (width 0.25) (layer "B.Cu") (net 20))
 (segment (start 134.68 65.97) (end 134.68 71.47) (width 0.25) (layer "B.Cu") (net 20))
 (segment (start 134.67 61.4) (end 135.845 62.575) (width 0.25) (layer "B.Cu") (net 20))
 (segment (start 135.845 64.805) (end 134.68 65.97) (width 0.25) (layer "B.Cu") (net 20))
 (segment (start 134.67 63.94) (end 132.15 66.46) (width 0.25) (layer "B.Cu") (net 19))
 (segment (start 132.15 66.46) (end 132.15 68.25) (width 0.25) (layer "B.Cu") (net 19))
 (segment (start 132.14 68.26) (end 132.14 71.47) (width 0.25) (layer "B.Cu") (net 19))
 (segment (start 132.15 68.25) (end 132.14 68.26) (width 0.25) (layer "B.Cu") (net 19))
 (segment (start 133.305 64.426701) (end 129.631701 68.1) (width 0.25) (layer "B.Cu") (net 18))
 (segment (start 129.6 68.1) (end 129.6 71.47) (width 0.25) (layer "B.Cu") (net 18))
 (segment (start 129.631701 68.1) (end 129.6 68.1) (width 0.25) (layer "B.Cu") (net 18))
 (segment (start 133.305 62.575) (end 133.305 64.426701) (width 0.25) (layer "B.Cu") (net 18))
 (segment (start 132.13 61.4) (end 133.305 62.575) (width 0.25) (layer "B.Cu") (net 18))
 (segment (start 132.13 63.94) (end 127.97 68.1) (width 0.25) (layer "B.Cu") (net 17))
 (segment (start 127.05 68.1) (end 127.06 68.11) (width 0.25) (layer "B.Cu") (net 17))
 (segment (start 127.06 68.11) (end 127.06 71.47) (width 0.25) (layer "B.Cu") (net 17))
 (segment (start 127.97 68.1) (end 127.05 68.1) (width 0.25) (layer "B.Cu") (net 17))
 (segment (start 130.765 64.435) (end 127.9 67.3) (width 0.25) (layer "B.Cu") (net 16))
 (segment (start 127.9 67.3) (end 124.55 67.3) (width 0.25) (layer "B.Cu") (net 16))
 (segment (start 130.765 62.575) (end 130.765 64.435) (width 0.25) (layer "B.Cu") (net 16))
 (segment (start 124.52 67.33) (end 124.52 71.47) (width 0.25) (layer "B.Cu") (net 16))
 (segment (start 124.55 67.3) (end 124.52 67.33) (width 0.25) (layer "B.Cu") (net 16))
 (segment (start 129.59 61.4) (end 130.765 62.575) (width 0.25) (layer "B.Cu") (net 16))
 (segment (start 122 66.4) (end 121.98 66.42) (width 0.25) (layer "B.Cu") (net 15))
 (segment (start 129.59 64.56) (end 127.75 66.4) (width 0.25) (layer "B.Cu") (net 15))
 (segment (start 129.59 63.94) (end 129.59 64.56) (width 0.25) (layer "B.Cu") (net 15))
 (segment (start 127.75 66.4) (end 122 66.4) (width 0.25) (layer "B.Cu") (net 15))
 (segment (start 121.98 66.42) (end 121.98 71.47) (width 0.25) (layer "B.Cu") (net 15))
 (segment (start 127.45 65.6) (end 119.45 65.6) (width 0.25) (layer "B.Cu") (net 14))
 (segment (start 119.44 65.61) (end 119.44 71.47) (width 0.25) (layer "B.Cu") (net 14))
 (segment (start 128.225 64.825) (end 127.45 65.6) (width 0.25) (layer "B.Cu") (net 14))
 (segment (start 127.05 61.4) (end 128.225 62.575) (width 0.25) (layer "B.Cu") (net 14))
 (segment (start 119.45 65.6) (end 119.44 65.61) (width 0.25) (layer "B.Cu") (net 14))
 (segment (start 128.225 62.575) (end 128.225 64.825) (width 0.25) (layer "B.Cu") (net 14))
 (segment (start 116.9 71.47) (end 116.9 64) (width 0.25) (layer "B.Cu") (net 13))
 (segment (start 116.9 64) (end 116.96 63.94) (width 0.25) (layer "B.Cu") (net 13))
 (segment (start 116.96 63.94) (end 127.05 63.94) (width 0.25) (layer "B.Cu") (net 13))
 (segment (start 149.92 92.806) (end 149.92 114.65) (width 0.25) (layer "B.Cu") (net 10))
 (segment (start 114.36 100.68) (end 114.36 92.806) (width 0.25) (layer "B.Cu") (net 10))
 (segment (start 114.36 92.806) (end 149.92 92.806) (width 0.25) (layer "B.Cu") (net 10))
 (segment (start 116.9 100.68) (end 114.36 100.68) (width 0.25) (layer "B.Cu") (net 10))
 (segment (start 116.9 98.14) (end 129.6 98.14) (width 0.25) (layer "B.Cu") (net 9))
 (segment (start 129.6 98.14) (end 129.6 114.65) (width 0.25) (layer "B.Cu") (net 9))
 (segment (start 121.98 143.86) (end 121.98 138.018) (width 0.25) (layer "B.Cu") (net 7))
 (segment (start 127.06 123.54) (end 123.25 123.54) (width 0.25) (layer "B.Cu") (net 7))
 (segment (start 123.25 138.018) (end 123.25 123.54) (width 0.25) (layer "B.Cu") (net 7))
 (segment (start 121.98 138.018) (end 123.25 138.018) (width 0.25) (layer "B.Cu") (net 7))
 (segment (start 127.06 114.65) (end 127.06 123.54) (width 0.25) (layer "B.Cu") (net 7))
 (segment (start 142.3 102.204) (end 124.52 102.204) (width 0.25) (layer "F.Cu") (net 34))
 (segment (start 142.3 86.71) (end 142.3 102.204) (width 0.25) (layer "F.Cu") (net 34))
 (segment (start 124.52 102.204) (end 124.52 114.65) (width 0.25) (layer "F.Cu") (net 34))
 (segment (start 121.98 100.934) (end 121.98 114.65) (width 0.25) (layer "F.Cu") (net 33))
 (segment (start 139.76 100.934) (end 121.98 100.934) (width 0.25) (layer "F.Cu") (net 33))
 (segment (start 139.76 86.71) (end 139.76 100.934) (width 0.25) (layer "F.Cu") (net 33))
 (segment (start 121.218 99.664) (end 121.218 112.872) (width 0.25) (layer "F.Cu") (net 32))
 (segment (start 137.22 86.71) (end 137.22 99.664) (width 0.25) (layer "F.Cu") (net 32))
 (segment (start 121.218 112.872) (end 119.44 114.65) (width 0.25) (layer "F.Cu") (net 32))
 (segment (start 137.22 99.664) (end 121.218 99.664) (width 0.25) (layer "F.Cu") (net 32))
 (segment (start 134.68 98.648) (end 120.456 98.648) (width 0.25) (layer "F.Cu") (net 31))
 (segment (start 116.9 112.11) (end 116.9 114.65) (width 0.25) (layer "F.Cu") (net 31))
 (segment (start 119.948 112.11) (end 116.9 112.11) (width 0.25) (layer "F.Cu") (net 31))
 (segment (start 134.68 86.71) (end 134.68 98.648) (width 0.25) (layer "F.Cu") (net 31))
 (segment (start 120.456 111.602) (end 119.948 112.11) (width 0.25) (layer "F.Cu") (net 31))
 (segment (start 120.456 98.648) (end 120.456 111.602) (width 0.25) (layer "F.Cu") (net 31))
 (segment (start 157.794 108.3) (end 139.76 108.3) (width 0.25) (layer "F.Cu") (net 11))
 (segment (start 157.784 101.96) (end 157.794 101.95) (width 0.25) (layer "F.Cu") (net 11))
 (segment (start 139.76 108.3) (end 139.76 114.65) (width 0.25) (layer "F.Cu") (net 11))
 (segment (start 155.025 101.96) (end 157.784 101.96) (width 0.25) (layer "F.Cu") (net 11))
 (segment (start 157.794 101.95) (end 157.794 108.3) (width 0.25) (layer "F.Cu") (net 11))
 (segment (start 146.11 104.49) (end 146.11 105.76) (width 0.25) (layer "F.Cu") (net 12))
 (segment (start 146.11 105.76) (end 137.22 105.76) (width 0.25) (layer "F.Cu") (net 12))
 (segment (start 155.025 104.5) (end 146.12 104.5) (width 0.25) (layer "F.Cu") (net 12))
 (segment (start 146.12 104.5) (end 146.11 104.49) (width 0.25) (layer "F.Cu") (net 12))
 (segment (start 137.22 105.76) (end 137.22 114.65) (width 0.25) (layer "F.Cu") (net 12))
 (segment (start 127.06 143.86) (end 127.06 129.89) (width 0.25) (layer "F.Cu") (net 5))
 (segment (start 124.52 143.86) (end 124.52 129.89) (width 0.25) (layer "F.Cu") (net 6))
 (segment (start 132.394 138.78) (end 132.14 138.526) (width 0.25) (layer "F.Cu") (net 2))
 (segment (start 149.92 143.86) (end 149.92 138.78) (width 0.25) (layer "F.Cu") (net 2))
 (segment (start 132.14 138.526) (end 132.14 129.89) (width 0.25) (layer "F.Cu") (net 2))
 (segment (start 149.92 138.78) (end 132.394 138.78) (width 0.25) (layer "F.Cu") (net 2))
 (segment (start 129.6 140.05) (end 129.6 129.89) (width 0.25) (layer "F.Cu") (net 4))
 (segment (start 142.3 143.86) (end 142.3 140.05) (width 0.25) (layer "F.Cu") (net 4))
 (segment (start 142.3 140.05) (end 129.6 140.05) (width 0.25) (layer "F.Cu") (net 4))
 (segment (start 134.68 95.6) (end 134.68 114.65) (width 0.25) (layer "B.Cu") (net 8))
 (segment (start 116.9 95.6) (end 134.68 95.6) (width 0.25) (layer "B.Cu") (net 8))
 (segment (start 128.33 103.474) (end 128.33 121) (width 0.25) (layer "F.Cu") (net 35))
 (segment (start 144.84 103.474) (end 128.33 103.474) (width 0.25) (layer "F.Cu") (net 35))
 (segment (start 144.84 86.71) (end 144.84 103.474) (width 0.25) (layer "F.Cu") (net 35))
 (segment (start 121.98 121) (end 121.98 129.89) (width 0.25) (layer "F.Cu") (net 35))
 (segment (start 128.33 121) (end 121.98 121) (width 0.25) (layer "F.Cu") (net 35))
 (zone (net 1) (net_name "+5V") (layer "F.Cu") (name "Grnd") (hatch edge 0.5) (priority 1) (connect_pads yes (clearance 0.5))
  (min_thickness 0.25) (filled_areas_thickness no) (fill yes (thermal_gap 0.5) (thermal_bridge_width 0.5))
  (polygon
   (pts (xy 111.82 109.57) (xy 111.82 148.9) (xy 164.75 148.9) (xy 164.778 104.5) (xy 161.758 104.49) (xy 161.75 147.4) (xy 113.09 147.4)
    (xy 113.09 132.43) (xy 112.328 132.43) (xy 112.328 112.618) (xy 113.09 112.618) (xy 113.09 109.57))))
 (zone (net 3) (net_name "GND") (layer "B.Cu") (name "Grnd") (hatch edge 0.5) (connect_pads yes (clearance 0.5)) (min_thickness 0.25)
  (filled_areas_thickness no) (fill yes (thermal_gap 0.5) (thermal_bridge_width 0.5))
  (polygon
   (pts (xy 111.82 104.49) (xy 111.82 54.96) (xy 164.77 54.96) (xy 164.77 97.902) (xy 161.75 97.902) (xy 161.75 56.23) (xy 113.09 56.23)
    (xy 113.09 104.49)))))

